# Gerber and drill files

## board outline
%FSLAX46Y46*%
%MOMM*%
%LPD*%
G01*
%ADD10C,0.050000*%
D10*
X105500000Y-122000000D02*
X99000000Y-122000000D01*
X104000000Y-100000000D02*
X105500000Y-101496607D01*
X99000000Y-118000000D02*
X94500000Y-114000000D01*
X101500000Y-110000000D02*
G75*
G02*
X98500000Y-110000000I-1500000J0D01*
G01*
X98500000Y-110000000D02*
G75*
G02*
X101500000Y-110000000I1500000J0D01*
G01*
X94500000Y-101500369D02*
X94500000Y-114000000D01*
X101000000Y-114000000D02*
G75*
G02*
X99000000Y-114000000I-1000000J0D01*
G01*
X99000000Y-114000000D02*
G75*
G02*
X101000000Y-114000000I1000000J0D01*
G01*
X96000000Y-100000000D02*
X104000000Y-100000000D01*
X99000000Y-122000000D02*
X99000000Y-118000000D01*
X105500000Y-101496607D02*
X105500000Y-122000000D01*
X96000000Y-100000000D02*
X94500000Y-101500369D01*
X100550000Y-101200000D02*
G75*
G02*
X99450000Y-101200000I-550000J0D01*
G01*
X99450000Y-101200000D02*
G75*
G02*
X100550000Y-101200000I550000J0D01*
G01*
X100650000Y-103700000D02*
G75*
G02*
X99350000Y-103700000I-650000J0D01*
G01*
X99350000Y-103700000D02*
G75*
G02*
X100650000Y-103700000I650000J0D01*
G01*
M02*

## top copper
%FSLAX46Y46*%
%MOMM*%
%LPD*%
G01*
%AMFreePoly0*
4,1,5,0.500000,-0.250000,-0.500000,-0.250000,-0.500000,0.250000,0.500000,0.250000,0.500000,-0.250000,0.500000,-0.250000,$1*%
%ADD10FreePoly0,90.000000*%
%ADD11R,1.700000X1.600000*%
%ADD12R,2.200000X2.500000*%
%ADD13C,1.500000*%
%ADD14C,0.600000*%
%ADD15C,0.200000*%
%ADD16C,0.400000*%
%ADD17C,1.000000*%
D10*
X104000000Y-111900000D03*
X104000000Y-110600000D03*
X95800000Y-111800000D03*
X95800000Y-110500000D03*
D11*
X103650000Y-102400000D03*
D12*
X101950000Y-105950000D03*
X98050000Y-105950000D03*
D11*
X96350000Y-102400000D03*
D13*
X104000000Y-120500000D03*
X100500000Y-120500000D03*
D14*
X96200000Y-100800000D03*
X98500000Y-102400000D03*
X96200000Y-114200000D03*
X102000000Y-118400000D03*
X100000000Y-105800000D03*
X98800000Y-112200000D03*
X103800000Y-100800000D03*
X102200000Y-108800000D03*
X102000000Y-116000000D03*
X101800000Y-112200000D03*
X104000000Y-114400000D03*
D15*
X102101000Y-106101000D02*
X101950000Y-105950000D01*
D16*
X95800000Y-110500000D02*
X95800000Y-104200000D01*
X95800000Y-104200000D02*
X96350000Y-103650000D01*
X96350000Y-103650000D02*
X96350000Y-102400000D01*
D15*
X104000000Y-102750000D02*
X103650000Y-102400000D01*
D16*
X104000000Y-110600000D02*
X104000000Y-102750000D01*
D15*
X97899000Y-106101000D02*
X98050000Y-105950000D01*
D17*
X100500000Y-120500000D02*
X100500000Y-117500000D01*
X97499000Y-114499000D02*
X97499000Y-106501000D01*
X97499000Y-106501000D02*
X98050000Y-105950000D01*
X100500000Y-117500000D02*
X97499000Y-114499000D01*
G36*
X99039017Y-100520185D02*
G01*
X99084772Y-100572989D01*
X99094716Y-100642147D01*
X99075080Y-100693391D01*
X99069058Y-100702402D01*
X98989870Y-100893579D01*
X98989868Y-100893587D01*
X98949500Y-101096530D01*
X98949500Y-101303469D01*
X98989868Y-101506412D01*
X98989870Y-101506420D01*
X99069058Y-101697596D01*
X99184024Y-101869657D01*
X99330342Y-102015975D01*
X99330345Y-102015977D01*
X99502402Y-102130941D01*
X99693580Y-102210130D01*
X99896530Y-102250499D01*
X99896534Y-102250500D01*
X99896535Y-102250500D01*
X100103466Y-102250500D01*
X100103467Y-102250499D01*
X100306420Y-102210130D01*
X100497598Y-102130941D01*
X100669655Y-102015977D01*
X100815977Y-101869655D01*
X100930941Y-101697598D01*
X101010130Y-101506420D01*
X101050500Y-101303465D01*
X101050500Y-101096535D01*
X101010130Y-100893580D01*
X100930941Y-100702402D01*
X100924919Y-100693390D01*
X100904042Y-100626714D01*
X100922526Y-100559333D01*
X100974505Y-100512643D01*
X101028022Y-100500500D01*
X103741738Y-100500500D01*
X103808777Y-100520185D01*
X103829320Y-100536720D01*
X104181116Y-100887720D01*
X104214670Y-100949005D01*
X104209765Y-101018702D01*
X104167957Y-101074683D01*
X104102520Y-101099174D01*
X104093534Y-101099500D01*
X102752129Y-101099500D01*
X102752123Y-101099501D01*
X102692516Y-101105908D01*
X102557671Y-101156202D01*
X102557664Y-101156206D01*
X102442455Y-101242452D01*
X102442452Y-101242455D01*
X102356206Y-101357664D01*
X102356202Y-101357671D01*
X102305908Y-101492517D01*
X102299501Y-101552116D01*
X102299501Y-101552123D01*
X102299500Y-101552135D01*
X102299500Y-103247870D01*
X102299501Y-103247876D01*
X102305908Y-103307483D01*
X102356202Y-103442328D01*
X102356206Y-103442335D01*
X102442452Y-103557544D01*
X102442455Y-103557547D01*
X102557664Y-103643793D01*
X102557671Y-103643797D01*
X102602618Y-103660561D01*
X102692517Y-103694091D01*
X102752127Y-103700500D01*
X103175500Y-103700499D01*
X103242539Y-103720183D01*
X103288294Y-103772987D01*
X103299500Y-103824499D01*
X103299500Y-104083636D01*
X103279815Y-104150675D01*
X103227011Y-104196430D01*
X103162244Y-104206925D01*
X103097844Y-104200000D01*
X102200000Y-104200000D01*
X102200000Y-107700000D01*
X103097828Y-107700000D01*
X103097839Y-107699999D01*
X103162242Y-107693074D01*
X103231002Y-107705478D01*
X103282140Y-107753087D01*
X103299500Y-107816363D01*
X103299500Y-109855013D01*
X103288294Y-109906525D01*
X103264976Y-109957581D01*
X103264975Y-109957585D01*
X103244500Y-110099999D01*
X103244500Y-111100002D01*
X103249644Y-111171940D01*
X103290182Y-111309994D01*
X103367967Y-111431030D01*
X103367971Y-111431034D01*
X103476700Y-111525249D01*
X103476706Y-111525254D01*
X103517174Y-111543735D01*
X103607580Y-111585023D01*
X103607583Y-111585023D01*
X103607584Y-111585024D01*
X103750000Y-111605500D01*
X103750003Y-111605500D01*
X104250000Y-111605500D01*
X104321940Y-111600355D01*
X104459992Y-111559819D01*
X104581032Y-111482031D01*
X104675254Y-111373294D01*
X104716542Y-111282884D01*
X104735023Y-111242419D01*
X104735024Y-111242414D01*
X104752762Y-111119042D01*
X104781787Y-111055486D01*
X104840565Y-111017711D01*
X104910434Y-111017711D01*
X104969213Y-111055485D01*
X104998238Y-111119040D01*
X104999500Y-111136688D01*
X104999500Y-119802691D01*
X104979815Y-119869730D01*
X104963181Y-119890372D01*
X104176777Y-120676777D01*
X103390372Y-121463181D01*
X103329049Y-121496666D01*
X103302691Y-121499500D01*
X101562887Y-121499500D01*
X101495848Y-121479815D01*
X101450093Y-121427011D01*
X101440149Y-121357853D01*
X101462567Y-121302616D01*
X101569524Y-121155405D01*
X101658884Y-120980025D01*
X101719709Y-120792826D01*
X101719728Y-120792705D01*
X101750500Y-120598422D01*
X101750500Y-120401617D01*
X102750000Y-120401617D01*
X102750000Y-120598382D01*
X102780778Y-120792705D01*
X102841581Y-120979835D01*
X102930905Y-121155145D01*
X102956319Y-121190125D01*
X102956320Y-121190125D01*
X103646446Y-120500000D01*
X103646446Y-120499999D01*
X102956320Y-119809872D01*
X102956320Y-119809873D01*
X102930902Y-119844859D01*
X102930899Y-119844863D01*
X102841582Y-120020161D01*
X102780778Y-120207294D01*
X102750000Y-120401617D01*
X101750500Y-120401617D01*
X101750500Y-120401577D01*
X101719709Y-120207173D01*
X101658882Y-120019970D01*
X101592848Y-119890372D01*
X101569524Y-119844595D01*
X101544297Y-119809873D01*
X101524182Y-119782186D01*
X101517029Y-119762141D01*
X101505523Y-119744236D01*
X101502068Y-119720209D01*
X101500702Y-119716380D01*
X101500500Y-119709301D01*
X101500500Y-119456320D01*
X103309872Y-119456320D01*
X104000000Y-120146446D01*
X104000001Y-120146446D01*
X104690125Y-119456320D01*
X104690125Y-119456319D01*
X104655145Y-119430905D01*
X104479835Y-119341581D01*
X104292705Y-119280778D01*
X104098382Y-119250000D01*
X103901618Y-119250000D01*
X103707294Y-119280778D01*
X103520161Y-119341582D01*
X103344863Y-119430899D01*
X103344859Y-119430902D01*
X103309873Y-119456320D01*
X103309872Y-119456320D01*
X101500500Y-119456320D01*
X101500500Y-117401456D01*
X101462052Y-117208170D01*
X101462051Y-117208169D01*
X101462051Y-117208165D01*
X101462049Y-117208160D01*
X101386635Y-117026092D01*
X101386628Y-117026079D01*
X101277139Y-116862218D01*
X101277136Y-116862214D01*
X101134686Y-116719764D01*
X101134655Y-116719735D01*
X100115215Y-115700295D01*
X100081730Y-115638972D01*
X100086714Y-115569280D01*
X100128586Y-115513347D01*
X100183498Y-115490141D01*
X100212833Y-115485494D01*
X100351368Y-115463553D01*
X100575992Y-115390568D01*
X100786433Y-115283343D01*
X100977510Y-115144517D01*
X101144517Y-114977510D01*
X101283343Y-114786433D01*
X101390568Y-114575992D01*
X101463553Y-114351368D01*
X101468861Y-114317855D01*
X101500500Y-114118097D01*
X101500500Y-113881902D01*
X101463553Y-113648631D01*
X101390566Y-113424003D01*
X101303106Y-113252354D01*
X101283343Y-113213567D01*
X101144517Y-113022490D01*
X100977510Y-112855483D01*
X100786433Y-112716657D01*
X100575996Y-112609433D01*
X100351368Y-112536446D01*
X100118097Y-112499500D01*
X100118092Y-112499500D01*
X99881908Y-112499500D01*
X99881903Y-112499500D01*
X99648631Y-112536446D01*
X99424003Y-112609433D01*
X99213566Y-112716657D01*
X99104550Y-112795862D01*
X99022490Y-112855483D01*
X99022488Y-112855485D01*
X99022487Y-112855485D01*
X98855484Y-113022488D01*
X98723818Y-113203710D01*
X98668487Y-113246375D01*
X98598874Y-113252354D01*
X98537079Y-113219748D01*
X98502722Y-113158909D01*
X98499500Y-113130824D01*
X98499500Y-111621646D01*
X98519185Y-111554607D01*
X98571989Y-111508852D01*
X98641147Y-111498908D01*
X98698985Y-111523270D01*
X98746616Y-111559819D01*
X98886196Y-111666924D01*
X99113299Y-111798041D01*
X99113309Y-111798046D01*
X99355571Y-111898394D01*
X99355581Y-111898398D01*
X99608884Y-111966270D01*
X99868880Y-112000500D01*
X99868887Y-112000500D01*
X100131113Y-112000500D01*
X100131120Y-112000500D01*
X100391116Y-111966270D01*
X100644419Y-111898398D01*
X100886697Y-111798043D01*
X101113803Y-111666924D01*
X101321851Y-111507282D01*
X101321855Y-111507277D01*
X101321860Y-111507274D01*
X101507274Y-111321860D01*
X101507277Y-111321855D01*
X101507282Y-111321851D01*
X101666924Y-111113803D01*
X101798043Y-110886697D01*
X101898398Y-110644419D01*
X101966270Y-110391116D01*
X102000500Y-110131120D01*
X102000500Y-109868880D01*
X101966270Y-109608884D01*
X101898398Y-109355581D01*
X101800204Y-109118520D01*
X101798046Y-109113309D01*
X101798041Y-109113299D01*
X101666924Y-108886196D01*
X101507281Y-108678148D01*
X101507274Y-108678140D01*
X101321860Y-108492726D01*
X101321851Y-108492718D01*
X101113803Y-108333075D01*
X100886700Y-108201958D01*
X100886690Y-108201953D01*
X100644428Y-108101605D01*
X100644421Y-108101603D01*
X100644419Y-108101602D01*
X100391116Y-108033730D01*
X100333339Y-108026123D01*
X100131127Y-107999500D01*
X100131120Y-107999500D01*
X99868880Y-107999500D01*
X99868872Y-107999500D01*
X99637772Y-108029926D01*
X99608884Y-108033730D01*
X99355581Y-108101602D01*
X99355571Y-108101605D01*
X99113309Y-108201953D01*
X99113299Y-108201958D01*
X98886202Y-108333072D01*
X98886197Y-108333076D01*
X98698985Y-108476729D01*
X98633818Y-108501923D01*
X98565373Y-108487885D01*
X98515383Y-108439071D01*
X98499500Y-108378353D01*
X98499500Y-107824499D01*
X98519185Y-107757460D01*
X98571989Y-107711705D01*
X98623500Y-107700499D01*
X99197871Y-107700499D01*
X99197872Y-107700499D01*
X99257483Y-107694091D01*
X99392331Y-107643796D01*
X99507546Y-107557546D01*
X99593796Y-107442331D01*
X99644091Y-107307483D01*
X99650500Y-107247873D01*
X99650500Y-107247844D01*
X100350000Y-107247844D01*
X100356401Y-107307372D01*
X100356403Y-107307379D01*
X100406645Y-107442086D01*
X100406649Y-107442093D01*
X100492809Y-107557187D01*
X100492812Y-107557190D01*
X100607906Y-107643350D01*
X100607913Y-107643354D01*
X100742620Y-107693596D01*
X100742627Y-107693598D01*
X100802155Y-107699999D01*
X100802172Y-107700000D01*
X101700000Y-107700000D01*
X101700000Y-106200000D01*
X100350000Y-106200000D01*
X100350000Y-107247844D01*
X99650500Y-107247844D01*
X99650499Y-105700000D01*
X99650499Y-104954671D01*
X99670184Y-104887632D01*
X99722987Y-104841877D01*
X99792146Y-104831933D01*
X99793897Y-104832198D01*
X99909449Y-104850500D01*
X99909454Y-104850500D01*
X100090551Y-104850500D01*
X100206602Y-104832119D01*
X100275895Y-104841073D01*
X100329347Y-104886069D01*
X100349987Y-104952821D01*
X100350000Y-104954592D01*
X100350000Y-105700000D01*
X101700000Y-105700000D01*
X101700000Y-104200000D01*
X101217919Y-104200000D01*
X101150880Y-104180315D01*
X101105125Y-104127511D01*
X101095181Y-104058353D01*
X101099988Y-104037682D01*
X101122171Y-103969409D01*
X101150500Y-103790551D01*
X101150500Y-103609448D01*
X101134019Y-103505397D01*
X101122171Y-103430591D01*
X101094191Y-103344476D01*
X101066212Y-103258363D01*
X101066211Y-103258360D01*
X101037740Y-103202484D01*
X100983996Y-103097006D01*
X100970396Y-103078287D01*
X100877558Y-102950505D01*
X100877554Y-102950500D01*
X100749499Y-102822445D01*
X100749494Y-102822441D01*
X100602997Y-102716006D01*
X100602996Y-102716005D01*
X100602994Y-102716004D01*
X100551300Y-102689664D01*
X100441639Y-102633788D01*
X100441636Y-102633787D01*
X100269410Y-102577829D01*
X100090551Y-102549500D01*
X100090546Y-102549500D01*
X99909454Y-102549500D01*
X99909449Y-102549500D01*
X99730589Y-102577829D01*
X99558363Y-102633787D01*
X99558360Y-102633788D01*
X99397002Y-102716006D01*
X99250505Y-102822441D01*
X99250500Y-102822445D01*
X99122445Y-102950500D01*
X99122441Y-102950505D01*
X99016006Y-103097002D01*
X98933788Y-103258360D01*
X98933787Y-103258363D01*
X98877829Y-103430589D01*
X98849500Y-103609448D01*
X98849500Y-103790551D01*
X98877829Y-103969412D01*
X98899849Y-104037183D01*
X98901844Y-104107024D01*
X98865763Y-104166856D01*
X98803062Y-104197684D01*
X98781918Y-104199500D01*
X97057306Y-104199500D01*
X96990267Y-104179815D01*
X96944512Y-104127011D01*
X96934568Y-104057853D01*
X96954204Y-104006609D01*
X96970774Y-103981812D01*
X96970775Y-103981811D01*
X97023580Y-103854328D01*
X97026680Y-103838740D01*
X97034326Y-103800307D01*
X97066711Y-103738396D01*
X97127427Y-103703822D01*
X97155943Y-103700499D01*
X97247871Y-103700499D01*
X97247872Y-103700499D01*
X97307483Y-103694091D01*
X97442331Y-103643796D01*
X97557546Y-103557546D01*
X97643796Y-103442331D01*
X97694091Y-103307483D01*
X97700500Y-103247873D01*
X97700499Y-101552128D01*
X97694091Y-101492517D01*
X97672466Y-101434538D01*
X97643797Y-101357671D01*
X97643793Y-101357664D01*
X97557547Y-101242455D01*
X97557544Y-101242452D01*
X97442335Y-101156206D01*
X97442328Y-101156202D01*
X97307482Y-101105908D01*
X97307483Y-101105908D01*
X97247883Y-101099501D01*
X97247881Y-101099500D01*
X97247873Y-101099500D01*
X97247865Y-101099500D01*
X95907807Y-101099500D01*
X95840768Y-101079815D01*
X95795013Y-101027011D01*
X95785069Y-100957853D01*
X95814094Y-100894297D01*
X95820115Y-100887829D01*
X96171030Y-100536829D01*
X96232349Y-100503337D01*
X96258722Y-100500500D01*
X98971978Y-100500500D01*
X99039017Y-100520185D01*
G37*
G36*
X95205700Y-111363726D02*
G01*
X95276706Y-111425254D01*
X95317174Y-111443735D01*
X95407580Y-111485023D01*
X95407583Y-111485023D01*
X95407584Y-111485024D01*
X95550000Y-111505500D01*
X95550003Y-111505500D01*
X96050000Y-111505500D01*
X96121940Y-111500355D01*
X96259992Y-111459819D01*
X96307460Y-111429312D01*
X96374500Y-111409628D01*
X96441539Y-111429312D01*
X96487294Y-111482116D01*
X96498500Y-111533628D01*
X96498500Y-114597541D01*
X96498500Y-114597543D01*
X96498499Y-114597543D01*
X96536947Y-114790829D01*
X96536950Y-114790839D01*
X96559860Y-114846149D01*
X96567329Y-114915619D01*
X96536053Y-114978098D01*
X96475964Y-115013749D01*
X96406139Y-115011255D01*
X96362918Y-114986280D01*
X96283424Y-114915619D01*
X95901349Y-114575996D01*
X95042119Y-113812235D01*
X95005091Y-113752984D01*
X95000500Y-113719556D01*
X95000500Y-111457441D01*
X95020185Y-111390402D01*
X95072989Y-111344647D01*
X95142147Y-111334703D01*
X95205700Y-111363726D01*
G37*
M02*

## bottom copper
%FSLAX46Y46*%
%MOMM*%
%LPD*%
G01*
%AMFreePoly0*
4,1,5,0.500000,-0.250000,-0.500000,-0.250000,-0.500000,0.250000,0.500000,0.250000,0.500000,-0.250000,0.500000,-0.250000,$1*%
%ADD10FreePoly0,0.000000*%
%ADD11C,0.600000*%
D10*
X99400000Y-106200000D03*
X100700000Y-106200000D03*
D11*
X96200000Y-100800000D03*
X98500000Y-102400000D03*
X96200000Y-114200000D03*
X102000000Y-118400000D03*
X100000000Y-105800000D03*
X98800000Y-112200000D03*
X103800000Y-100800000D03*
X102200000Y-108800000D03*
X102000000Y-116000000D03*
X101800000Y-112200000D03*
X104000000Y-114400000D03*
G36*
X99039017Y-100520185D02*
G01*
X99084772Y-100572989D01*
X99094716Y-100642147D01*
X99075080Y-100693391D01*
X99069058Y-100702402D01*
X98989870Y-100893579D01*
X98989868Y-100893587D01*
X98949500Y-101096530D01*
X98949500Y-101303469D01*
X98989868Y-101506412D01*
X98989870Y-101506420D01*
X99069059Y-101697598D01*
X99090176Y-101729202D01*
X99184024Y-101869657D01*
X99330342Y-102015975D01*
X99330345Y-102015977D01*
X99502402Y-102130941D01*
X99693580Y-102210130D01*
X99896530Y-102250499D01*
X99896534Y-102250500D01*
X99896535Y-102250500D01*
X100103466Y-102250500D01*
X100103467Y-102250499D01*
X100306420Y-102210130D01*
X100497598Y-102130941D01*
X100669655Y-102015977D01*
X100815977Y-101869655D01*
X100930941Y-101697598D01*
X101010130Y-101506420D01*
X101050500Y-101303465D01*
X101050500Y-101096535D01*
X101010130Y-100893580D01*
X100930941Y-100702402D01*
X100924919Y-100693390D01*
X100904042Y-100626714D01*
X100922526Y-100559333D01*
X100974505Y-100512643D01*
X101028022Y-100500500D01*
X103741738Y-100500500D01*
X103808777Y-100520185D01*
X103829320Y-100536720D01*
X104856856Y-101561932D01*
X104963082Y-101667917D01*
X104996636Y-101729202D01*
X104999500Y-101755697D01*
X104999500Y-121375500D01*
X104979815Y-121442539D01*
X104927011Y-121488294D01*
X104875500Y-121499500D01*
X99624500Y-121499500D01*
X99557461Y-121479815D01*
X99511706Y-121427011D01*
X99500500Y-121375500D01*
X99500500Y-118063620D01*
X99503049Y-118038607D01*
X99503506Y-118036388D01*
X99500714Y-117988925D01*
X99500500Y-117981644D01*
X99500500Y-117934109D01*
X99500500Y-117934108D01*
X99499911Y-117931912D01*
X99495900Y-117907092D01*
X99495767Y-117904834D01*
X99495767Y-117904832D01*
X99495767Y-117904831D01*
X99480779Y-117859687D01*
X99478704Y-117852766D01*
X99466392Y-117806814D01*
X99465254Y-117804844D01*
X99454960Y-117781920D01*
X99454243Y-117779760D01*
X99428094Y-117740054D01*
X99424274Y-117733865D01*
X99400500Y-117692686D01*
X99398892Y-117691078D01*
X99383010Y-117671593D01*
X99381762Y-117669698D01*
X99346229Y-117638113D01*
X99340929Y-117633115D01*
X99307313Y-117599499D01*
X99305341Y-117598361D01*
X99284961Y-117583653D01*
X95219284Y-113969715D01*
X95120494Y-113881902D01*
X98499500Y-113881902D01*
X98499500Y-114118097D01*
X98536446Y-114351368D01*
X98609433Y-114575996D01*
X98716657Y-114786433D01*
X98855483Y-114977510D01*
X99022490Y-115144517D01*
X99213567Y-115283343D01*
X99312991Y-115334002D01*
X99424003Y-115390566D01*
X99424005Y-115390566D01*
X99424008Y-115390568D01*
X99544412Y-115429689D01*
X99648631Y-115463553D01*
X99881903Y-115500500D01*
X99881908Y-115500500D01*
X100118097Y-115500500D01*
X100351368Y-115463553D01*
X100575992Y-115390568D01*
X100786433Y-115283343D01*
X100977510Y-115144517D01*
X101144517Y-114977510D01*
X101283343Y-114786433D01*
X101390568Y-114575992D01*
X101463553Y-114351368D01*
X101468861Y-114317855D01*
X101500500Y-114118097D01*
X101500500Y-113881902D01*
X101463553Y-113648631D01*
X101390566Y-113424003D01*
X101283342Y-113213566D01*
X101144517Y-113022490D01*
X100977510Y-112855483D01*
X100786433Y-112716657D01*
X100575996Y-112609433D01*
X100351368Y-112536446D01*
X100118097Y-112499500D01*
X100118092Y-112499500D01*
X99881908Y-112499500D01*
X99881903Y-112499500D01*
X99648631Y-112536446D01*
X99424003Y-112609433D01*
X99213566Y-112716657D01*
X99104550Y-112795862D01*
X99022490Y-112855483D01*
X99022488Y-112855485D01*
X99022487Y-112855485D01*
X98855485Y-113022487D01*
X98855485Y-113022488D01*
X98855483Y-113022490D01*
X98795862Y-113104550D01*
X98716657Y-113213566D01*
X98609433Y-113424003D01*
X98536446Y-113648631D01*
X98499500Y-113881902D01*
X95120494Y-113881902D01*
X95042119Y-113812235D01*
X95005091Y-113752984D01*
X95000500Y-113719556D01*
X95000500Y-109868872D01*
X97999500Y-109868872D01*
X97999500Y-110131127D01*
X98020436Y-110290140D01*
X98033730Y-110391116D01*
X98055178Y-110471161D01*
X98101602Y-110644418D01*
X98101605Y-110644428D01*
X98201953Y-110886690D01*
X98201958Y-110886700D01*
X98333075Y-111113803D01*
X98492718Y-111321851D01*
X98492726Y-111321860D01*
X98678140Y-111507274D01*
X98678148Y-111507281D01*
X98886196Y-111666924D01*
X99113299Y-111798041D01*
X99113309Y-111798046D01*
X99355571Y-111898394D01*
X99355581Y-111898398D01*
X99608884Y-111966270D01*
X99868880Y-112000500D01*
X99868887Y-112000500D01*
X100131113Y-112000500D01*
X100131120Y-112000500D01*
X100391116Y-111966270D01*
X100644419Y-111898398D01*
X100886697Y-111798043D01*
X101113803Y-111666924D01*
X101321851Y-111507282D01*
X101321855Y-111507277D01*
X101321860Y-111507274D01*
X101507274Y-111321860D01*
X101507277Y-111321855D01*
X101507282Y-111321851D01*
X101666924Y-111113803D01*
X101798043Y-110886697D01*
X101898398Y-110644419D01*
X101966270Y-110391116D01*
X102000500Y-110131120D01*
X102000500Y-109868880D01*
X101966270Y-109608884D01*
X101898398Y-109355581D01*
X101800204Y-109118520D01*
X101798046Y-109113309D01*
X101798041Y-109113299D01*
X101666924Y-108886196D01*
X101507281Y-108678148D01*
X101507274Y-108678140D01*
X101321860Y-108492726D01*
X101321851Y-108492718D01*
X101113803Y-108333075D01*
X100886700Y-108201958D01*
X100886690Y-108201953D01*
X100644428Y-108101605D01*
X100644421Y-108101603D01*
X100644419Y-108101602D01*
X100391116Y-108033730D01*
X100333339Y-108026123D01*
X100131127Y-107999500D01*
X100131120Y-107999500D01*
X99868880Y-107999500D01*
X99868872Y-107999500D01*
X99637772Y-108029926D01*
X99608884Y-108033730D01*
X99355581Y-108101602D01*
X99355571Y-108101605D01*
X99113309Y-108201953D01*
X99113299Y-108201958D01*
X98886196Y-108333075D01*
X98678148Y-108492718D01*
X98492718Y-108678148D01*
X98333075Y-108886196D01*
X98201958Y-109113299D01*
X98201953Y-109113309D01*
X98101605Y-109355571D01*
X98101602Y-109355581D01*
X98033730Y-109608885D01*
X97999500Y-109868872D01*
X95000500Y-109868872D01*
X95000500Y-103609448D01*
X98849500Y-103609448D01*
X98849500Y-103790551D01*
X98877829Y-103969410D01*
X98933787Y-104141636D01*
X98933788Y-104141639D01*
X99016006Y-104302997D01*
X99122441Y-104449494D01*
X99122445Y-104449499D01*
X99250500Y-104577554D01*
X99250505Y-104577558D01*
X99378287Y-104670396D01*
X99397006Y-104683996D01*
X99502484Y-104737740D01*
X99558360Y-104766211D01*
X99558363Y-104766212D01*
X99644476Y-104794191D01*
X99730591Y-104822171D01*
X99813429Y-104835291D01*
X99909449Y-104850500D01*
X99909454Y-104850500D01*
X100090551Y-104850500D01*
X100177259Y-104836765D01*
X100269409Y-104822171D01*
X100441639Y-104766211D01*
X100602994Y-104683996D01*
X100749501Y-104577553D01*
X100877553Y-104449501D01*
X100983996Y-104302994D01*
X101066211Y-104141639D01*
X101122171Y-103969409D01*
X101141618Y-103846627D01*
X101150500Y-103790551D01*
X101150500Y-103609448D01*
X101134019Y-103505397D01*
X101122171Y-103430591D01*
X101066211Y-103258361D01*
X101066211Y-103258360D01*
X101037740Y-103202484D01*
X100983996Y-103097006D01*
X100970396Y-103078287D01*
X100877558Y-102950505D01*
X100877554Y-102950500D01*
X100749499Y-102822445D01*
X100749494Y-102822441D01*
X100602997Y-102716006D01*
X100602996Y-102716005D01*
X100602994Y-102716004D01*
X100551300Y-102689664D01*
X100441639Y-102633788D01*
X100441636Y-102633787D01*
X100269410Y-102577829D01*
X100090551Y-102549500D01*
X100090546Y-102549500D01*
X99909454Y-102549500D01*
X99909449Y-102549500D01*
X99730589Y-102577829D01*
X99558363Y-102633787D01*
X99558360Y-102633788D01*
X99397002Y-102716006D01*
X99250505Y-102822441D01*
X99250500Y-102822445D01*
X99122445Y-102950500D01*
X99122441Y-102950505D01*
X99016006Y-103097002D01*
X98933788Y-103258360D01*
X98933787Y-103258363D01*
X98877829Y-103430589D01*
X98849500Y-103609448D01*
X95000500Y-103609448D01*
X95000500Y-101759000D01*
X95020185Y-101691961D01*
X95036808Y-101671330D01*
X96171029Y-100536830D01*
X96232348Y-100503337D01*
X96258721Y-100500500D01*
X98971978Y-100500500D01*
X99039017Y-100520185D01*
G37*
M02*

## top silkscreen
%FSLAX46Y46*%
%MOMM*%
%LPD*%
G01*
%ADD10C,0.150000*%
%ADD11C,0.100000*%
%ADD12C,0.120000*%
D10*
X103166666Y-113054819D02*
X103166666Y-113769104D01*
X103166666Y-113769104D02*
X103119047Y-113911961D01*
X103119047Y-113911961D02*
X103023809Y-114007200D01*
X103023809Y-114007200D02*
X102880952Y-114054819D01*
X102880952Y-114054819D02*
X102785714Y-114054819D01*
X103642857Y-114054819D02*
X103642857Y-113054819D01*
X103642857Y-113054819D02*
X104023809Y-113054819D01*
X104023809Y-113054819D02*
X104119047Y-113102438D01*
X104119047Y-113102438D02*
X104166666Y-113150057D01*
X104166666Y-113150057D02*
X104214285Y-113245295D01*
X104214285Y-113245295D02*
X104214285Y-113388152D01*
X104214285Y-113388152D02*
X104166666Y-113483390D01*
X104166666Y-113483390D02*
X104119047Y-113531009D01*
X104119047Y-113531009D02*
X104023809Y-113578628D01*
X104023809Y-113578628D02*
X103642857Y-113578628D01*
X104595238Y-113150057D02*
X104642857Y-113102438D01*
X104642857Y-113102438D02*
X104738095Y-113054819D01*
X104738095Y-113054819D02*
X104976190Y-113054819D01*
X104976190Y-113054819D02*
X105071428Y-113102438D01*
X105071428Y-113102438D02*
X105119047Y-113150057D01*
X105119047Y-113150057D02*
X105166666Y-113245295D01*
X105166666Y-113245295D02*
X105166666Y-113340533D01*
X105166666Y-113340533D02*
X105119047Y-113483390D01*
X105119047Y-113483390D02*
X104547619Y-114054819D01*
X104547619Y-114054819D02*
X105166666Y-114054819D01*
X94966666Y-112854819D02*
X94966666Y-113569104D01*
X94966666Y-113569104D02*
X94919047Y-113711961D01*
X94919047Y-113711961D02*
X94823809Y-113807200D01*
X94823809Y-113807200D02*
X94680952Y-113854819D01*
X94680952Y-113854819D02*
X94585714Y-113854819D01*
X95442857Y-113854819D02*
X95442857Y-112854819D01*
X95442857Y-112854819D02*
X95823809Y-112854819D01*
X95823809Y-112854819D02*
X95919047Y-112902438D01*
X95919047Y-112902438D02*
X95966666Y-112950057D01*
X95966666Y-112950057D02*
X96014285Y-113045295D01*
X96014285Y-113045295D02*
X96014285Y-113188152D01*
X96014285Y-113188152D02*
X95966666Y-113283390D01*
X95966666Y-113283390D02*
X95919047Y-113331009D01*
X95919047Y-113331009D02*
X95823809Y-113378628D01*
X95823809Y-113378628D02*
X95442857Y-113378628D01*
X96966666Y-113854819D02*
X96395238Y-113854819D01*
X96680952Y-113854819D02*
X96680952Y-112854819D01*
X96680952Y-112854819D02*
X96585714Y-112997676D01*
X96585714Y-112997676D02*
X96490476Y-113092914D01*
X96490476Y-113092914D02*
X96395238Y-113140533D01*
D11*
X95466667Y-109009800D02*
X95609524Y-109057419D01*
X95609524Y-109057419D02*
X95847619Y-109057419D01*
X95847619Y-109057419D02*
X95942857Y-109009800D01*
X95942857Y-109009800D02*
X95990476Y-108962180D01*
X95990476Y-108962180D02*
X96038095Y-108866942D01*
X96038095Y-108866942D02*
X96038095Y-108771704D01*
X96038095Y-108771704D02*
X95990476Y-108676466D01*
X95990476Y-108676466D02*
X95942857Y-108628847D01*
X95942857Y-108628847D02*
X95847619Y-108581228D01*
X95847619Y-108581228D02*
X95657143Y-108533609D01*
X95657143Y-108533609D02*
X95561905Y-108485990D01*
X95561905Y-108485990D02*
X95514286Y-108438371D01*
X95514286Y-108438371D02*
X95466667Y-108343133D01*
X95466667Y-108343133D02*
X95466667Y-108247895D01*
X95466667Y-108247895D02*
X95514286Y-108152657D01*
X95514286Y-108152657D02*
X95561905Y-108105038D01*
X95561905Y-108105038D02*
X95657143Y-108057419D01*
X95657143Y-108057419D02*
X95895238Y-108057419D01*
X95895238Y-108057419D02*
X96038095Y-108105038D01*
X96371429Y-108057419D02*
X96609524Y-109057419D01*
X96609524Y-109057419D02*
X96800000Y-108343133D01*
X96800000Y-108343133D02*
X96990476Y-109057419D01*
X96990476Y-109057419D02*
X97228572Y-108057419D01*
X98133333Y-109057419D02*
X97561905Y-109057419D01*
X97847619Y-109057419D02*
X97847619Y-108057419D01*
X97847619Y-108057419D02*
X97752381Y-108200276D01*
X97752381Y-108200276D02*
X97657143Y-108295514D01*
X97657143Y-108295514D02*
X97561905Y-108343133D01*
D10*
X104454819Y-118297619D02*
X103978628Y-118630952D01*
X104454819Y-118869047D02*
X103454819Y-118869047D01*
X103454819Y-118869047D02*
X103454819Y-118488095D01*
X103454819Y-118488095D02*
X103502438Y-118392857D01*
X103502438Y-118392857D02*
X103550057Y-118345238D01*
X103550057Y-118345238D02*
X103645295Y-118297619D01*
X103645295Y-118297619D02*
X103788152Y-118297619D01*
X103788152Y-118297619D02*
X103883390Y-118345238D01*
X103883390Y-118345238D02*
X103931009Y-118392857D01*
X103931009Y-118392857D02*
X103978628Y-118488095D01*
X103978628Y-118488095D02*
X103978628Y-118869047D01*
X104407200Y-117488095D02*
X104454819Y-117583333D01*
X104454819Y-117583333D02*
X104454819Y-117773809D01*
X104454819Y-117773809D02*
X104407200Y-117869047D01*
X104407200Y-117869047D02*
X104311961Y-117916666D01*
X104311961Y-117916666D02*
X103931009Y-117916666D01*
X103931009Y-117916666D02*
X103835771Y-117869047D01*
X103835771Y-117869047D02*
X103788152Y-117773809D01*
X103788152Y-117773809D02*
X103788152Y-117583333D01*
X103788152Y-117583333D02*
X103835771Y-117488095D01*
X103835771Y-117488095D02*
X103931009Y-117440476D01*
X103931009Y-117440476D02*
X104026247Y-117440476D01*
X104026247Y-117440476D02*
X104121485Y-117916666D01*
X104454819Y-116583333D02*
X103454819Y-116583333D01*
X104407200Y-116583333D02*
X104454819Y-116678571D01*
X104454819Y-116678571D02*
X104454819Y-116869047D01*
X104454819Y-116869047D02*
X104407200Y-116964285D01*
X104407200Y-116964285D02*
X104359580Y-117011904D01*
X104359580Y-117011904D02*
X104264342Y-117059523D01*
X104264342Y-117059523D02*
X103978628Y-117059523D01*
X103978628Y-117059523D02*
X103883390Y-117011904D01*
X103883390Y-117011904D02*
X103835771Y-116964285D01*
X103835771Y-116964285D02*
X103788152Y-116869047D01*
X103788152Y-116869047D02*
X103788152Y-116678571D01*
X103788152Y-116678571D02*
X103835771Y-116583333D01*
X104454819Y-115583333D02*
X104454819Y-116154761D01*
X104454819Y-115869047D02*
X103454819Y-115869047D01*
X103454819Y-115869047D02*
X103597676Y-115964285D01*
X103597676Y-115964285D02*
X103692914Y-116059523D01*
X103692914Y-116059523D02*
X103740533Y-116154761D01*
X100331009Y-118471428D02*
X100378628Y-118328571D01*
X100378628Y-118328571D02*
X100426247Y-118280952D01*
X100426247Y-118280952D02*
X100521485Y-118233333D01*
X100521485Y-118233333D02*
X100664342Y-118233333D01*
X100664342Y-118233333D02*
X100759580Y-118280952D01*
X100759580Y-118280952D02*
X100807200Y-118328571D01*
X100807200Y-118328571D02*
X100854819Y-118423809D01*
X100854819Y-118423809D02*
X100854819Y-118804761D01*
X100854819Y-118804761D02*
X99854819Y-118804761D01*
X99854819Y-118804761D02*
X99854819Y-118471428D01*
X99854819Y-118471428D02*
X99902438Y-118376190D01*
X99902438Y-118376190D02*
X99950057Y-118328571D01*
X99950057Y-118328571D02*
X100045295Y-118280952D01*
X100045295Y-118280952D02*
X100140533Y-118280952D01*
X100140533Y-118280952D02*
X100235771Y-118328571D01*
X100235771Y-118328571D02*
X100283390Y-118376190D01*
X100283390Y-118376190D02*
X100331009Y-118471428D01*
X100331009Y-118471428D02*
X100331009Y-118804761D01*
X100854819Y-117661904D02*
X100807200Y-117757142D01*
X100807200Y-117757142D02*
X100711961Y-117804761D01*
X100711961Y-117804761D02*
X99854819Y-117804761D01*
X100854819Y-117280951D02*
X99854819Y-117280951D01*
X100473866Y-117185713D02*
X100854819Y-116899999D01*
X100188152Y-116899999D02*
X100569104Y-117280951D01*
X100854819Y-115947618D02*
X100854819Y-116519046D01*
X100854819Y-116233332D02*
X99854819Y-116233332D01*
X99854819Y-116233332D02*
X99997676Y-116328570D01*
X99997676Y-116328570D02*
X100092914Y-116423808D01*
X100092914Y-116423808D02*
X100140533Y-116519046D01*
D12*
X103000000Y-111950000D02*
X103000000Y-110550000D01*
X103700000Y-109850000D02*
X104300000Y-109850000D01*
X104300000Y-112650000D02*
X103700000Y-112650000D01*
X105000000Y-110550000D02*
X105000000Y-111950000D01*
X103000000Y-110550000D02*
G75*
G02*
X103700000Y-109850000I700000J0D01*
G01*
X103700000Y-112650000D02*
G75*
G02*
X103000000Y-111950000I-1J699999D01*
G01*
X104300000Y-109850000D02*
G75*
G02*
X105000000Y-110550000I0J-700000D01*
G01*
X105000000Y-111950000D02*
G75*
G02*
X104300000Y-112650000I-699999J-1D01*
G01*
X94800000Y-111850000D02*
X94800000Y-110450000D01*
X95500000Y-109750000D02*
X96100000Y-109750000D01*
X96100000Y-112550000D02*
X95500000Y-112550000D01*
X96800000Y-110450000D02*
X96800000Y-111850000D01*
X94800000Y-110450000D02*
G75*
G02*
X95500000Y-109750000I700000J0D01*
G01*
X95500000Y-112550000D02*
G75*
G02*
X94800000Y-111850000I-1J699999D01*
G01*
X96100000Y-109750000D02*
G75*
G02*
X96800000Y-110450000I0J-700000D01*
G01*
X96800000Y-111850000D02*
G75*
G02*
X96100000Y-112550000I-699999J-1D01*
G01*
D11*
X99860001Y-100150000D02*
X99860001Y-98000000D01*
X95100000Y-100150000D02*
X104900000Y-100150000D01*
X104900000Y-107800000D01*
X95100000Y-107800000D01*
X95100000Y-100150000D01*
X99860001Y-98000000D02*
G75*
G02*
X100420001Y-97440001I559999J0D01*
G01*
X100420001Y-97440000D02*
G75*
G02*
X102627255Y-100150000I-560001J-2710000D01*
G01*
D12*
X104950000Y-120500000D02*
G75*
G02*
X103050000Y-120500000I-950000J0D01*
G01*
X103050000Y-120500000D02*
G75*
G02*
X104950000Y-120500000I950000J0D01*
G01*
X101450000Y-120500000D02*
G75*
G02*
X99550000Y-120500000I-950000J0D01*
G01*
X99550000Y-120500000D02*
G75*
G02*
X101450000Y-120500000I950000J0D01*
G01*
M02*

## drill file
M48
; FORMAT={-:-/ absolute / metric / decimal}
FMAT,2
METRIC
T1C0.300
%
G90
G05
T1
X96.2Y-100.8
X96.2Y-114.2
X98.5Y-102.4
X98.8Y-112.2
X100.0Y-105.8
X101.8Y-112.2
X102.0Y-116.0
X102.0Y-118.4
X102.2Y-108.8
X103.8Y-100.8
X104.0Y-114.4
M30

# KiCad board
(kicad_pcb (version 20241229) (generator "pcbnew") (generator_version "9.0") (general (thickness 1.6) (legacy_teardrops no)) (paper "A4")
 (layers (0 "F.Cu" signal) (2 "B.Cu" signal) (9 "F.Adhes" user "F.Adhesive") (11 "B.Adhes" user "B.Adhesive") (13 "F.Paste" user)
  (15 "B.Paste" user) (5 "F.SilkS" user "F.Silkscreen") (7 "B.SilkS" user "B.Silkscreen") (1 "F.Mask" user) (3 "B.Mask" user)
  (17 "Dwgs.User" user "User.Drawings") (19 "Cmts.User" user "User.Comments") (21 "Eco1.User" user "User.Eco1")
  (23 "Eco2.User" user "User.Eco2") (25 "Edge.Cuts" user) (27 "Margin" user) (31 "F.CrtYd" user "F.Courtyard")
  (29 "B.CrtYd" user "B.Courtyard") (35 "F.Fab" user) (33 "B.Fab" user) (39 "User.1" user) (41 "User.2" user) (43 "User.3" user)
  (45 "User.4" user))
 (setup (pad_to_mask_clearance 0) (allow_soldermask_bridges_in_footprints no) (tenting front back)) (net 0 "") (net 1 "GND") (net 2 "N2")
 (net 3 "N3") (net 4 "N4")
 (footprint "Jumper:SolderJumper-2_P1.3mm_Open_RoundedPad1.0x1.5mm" (layer "F.Cu") (at 104 111.25 90)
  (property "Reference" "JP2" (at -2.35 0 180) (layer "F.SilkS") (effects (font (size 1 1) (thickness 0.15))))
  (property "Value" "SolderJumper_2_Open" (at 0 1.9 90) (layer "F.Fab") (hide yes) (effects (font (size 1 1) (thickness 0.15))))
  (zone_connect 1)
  (fp_line (start -0.7 -1) (end 0.7 -1) (stroke (width 0.12) (type solid)) (layer "F.SilkS"))
  (fp_line (start 1.4 -0.3) (end 1.4 0.3) (stroke (width 0.12) (type solid)) (layer "F.SilkS"))
  (fp_line (start -1.4 0.3) (end -1.4 -0.3) (stroke (width 0.12) (type solid)) (layer "F.SilkS"))
  (fp_line (start 0.7 1) (end -0.7 1) (stroke (width 0.12) (type solid)) (layer "F.SilkS"))
  (fp_arc (start 0.7 -1) (mid 1.194975 -0.794975) (end 1.4 -0.3) (stroke (width 0.12) (type solid)) (layer "F.SilkS"))
  (fp_arc (start -1.4 -0.3) (mid -1.194975 -0.794975) (end -0.7 -1) (stroke (width 0.12) (type solid)) (layer "F.SilkS"))
  (fp_arc (start 1.4 0.3) (mid 1.194975 0.794975) (end 0.7 1) (stroke (width 0.12) (type solid)) (layer "F.SilkS"))
  (fp_arc (start -0.7 1) (mid -1.194975 0.794975) (end -1.4 0.3) (stroke (width 0.12) (type solid)) (layer "F.SilkS"))
  (pad "1" smd custom (at -0.65 0 90) (size 1 0.5) (layers "F.Cu" "F.Mask") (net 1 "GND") (zone_connect 2) (thermal_bridge_angle 45)
   (options (clearance outline) (anchor rect)) (primitives))
  (pad "2" smd custom (at 0.65 0 90) (size 1 0.5) (layers "F.Cu" "F.Mask") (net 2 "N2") (zone_connect 2) (thermal_bridge_angle 45)
   (options (clearance outline) (anchor rect)) (primitives)))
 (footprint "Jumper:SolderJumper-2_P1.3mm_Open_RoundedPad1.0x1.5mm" (layer "F.Cu") (at 95.8 111.15 90)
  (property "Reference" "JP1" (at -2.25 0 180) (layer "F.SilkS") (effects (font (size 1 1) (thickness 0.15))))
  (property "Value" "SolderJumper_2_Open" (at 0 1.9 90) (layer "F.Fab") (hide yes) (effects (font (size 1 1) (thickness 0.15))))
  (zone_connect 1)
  (fp_line (start -0.7 -1) (end 0.7 -1) (stroke (width 0.12) (type solid)) (layer "F.SilkS"))
  (fp_line (start 1.4 -0.3) (end 1.4 0.3) (stroke (width 0.12) (type solid)) (layer "F.SilkS"))
  (fp_line (start -1.4 0.3) (end -1.4 -0.3) (stroke (width 0.12) (type solid)) (layer "F.SilkS"))
  (fp_line (start 0.7 1) (end -0.7 1) (stroke (width 0.12) (type solid)) (layer "F.SilkS"))
  (fp_arc (start 0.7 -1) (mid 1.194975 -0.794975) (end 1.4 -0.3) (stroke (width 0.12) (type solid)) (layer "F.SilkS"))
  (fp_arc (start -1.4 -0.3) (mid -1.194975 -0.794975) (end -0.7 -1) (stroke (width 0.12) (type solid)) (layer "F.SilkS"))
  (fp_arc (start 1.4 0.3) (mid 1.194975 0.794975) (end 0.7 1) (stroke (width 0.12) (type solid)) (layer "F.SilkS"))
  (fp_arc (start -0.7 1) (mid -1.194975 0.794975) (end -1.4 0.3) (stroke (width 0.12) (type solid)) (layer "F.SilkS"))
  (pad "1" smd custom (at -0.65 0 90) (size 1 0.5) (layers "F.Cu" "F.Mask") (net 1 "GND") (zone_connect 2) (thermal_bridge_angle 45)
   (options (clearance outline) (anchor rect)) (primitives))
  (pad "2" smd custom (at 0.65 0 90) (size 1 0.5) (layers "F.Cu" "F.Mask") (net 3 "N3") (zone_connect 2) (thermal_bridge_angle 45)
   (options (clearance outline) (anchor rect)) (primitives)))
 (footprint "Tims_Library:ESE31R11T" (layer "F.Cu") (at 100 101.2)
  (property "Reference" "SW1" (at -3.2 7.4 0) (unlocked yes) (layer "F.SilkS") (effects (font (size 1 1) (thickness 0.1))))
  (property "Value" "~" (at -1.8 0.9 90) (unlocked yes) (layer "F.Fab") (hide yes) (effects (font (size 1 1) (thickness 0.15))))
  (fp_line (start -0.139999 -1.05) (end -0.139999 -3.2) (stroke (width 0.1) (type default)) (layer "F.SilkS"))
  (fp_rect (start -4.9 -1.05) (end 4.9 6.6) (stroke (width 0.1) (type default)) (fill no) (layer "F.SilkS"))
  (fp_arc (start -0.139999 -3.2) (mid 0.024021 -3.59598) (end 0.420001 -3.76) (stroke (width 0.1) (type default)) (layer "F.SilkS"))
  (fp_arc (start 0.420001 -3.76) (mid 2.00562 -2.797575) (end 2.627256 -1.05) (stroke (width 0.1) (type default)) (layer "F.SilkS"))
  (fp_circle (center 0 0) (end 0 -0.55) (stroke (width 0.05) (type default)) (fill no) (layer "Edge.Cuts"))
  (fp_circle (center 0 2.5) (end 0 1.85) (stroke (width 0.05) (type default)) (fill no) (layer "Edge.Cuts"))
  (pad "1" smd rect (at 3.65 1.2) (size 1.7 1.6) (layers "F.Cu" "F.Mask" "F.Paste") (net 2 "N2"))
  (pad "2" smd rect (at 1.95 4.75) (size 2.2 2.5) (layers "F.Cu" "F.Mask" "F.Paste") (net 1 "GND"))
  (pad "3" smd rect (at -1.95 4.75) (size 2.2 2.5) (layers "F.Cu" "F.Mask" "F.Paste") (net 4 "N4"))
  (pad "4" smd rect (at -3.65 1.2) (size 1.7 1.6) (layers "F.Cu" "F.Mask" "F.Paste") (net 3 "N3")))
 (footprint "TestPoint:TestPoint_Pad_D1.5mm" (layer "F.Cu") (at 104 120.5 -90)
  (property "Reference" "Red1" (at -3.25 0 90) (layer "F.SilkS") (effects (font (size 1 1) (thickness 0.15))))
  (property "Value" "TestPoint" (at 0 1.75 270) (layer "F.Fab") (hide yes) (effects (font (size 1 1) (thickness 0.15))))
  (fp_circle (center 0 0) (end 0 0.95) (stroke (width 0.12) (type solid)) (fill no) (layer "F.SilkS"))
  (pad "1" smd circle (at 0 0 270) (size 1.5 1.5) (layers "F.Cu" "F.Mask") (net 1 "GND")))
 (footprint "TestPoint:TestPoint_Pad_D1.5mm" (layer "F.Cu") (at 100.5 120.5 -90)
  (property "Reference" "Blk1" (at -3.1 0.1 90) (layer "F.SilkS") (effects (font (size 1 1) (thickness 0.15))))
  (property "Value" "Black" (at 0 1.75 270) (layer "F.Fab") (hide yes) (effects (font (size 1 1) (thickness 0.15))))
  (fp_circle (center 0 0) (end 0 0.95) (stroke (width 0.12) (type solid)) (fill no) (layer "F.SilkS"))
  (pad "1" smd circle (at 0 0 270) (size 1.5 1.5) (layers "F.Cu" "F.Mask") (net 4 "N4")))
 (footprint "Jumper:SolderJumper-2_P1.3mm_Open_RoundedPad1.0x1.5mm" (layer "B.Cu") (at 100.05 106.2)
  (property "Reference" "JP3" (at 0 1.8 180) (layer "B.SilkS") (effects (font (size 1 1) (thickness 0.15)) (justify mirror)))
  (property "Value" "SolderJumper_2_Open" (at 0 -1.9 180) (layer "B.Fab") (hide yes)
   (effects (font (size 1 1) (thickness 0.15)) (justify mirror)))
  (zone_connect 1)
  (pad "1" smd custom (at -0.65 0) (size 1 0.5) (layers "B.Cu" "B.Mask") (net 1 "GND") (zone_connect 2) (thermal_bridge_angle 45)
   (options (clearance outline) (anchor rect)) (primitives))
  (pad "2" smd custom (at 0.65 0) (size 1 0.5) (layers "B.Cu" "B.Mask") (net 1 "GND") (zone_connect 2) (thermal_bridge_angle 45)
   (options (clearance outline) (anchor rect)) (primitives)))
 (gr_line (start 105.5 122) (end 99 122) (stroke (width 0.05) (type default)) (layer "Edge.Cuts"))
 (gr_line (start 104 100) (end 105.5 101.496607) (stroke (width 0.05) (type default)) (layer "Edge.Cuts"))
 (gr_line (start 99 118) (end 94.5 114) (stroke (width 0.05) (type default)) (layer "Edge.Cuts"))
 (gr_circle (center 100 110) (end 98.5 110) (stroke (width 0.05) (type default)) (fill no) (layer "Edge.Cuts"))
 (gr_line (start 94.5 101.500369) (end 94.5 114) (stroke (width 0.05) (type default)) (layer "Edge.Cuts"))
 (gr_circle (center 100 114) (end 100 115) (stroke (width 0.05) (type default)) (fill no) (layer "Edge.Cuts"))
 (gr_line (start 96 100) (end 104 100) (stroke (width 0.05) (type default)) (layer "Edge.Cuts"))
 (gr_line (start 99 122) (end 99 118) (stroke (width 0.05) (type default)) (layer "Edge.Cuts"))
 (gr_line (start 105.5 101.496607) (end 105.5 122) (stroke (width 0.05) (type default)) (layer "Edge.Cuts"))
 (gr_line (start 96 100) (end 94.5 101.500369) (stroke (width 0.05) (type default)) (layer "Edge.Cuts"))
 (segment (start 102.101 106.101) (end 101.95 105.95) (width 0.2) (layer "F.Cu") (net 1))
 (via (at 96.2 100.8) (size 0.6) (drill 0.3) (layers "F.Cu" "B.Cu") (free yes) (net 1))
 (via (at 98.5 102.4) (size 0.6) (drill 0.3) (layers "F.Cu" "B.Cu") (free yes) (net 1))
 (via (at 96.2 114.2) (size 0.6) (drill 0.3) (layers "F.Cu" "B.Cu") (free yes) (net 1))
 (via (at 102 118.4) (size 0.6) (drill 0.3) (layers "F.Cu" "B.Cu") (free yes) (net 1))
 (via (at 100 105.8) (size 0.6) (drill 0.3) (layers "F.Cu" "B.Cu") (free yes) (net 1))
 (via (at 98.8 112.2) (size 0.6) (drill 0.3) (layers "F.Cu" "B.Cu") (free yes) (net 1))
 (via (at 103.8 100.8) (size 0.6) (drill 0.3) (layers "F.Cu" "B.Cu") (free yes) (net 1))
 (via (at 102.2 108.8) (size 0.6) (drill 0.3) (layers "F.Cu" "B.Cu") (free yes) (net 1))
 (via (at 102 116) (size 0.6) (drill 0.3) (layers "F.Cu" "B.Cu") (free yes) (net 1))
 (via (at 101.8 112.2) (size 0.6) (drill 0.3) (layers "F.Cu" "B.Cu") (free yes) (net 1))
 (via (at 104 114.4) (size 0.6) (drill 0.3) (layers "F.Cu" "B.Cu") (free yes) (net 1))
 (segment (start 95.8 110.5) (end 95.8 104.2) (width 0.4) (layer "F.Cu") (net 3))
 (segment (start 95.8 104.2) (end 96.35 103.65) (width 0.4) (layer "F.Cu") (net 3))
 (segment (start 96.35 103.65) (end 96.35 102.4) (width 0.4) (layer "F.Cu") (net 3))
 (segment (start 104 102.75) (end 103.65 102.4) (width 0.2) (layer "F.Cu") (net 2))
 (segment (start 104 110.6) (end 104 102.75) (width 0.4) (layer "F.Cu") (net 2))
 (segment (start 97.899 106.101) (end 98.05 105.95) (width 0.2) (layer "F.Cu") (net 4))
 (segment (start 100.5 120.5) (end 100.5 117.5) (width 1) (layer "F.Cu") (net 4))
 (segment (start 97.499 114.499) (end 97.499 106.501) (width 1) (layer "F.Cu") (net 4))
 (segment (start 97.499 106.501) (end 98.05 105.95) (width 1) (layer "F.Cu") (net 4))
 (segment (start 100.5 117.5) (end 97.499 114.499) (width 1) (layer "F.Cu") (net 4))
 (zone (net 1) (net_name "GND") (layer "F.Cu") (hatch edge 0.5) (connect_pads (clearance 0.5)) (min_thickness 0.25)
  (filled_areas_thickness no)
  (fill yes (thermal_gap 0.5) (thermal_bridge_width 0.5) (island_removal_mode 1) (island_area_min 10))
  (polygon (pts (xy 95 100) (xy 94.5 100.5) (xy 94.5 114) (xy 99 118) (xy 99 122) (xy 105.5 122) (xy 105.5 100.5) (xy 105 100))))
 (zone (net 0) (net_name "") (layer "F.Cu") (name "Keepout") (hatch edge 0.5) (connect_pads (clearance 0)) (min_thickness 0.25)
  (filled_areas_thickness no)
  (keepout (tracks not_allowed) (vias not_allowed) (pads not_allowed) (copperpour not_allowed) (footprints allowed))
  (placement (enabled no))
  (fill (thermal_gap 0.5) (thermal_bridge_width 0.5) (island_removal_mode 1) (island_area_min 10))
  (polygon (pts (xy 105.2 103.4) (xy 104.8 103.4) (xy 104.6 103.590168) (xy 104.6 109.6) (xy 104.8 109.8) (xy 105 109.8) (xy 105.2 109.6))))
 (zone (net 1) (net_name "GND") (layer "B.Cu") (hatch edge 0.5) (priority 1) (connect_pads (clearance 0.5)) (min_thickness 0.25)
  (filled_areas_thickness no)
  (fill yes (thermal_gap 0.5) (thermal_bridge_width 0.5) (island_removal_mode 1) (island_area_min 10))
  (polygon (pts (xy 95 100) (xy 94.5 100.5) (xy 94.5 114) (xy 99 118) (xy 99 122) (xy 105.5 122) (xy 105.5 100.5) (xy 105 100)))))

